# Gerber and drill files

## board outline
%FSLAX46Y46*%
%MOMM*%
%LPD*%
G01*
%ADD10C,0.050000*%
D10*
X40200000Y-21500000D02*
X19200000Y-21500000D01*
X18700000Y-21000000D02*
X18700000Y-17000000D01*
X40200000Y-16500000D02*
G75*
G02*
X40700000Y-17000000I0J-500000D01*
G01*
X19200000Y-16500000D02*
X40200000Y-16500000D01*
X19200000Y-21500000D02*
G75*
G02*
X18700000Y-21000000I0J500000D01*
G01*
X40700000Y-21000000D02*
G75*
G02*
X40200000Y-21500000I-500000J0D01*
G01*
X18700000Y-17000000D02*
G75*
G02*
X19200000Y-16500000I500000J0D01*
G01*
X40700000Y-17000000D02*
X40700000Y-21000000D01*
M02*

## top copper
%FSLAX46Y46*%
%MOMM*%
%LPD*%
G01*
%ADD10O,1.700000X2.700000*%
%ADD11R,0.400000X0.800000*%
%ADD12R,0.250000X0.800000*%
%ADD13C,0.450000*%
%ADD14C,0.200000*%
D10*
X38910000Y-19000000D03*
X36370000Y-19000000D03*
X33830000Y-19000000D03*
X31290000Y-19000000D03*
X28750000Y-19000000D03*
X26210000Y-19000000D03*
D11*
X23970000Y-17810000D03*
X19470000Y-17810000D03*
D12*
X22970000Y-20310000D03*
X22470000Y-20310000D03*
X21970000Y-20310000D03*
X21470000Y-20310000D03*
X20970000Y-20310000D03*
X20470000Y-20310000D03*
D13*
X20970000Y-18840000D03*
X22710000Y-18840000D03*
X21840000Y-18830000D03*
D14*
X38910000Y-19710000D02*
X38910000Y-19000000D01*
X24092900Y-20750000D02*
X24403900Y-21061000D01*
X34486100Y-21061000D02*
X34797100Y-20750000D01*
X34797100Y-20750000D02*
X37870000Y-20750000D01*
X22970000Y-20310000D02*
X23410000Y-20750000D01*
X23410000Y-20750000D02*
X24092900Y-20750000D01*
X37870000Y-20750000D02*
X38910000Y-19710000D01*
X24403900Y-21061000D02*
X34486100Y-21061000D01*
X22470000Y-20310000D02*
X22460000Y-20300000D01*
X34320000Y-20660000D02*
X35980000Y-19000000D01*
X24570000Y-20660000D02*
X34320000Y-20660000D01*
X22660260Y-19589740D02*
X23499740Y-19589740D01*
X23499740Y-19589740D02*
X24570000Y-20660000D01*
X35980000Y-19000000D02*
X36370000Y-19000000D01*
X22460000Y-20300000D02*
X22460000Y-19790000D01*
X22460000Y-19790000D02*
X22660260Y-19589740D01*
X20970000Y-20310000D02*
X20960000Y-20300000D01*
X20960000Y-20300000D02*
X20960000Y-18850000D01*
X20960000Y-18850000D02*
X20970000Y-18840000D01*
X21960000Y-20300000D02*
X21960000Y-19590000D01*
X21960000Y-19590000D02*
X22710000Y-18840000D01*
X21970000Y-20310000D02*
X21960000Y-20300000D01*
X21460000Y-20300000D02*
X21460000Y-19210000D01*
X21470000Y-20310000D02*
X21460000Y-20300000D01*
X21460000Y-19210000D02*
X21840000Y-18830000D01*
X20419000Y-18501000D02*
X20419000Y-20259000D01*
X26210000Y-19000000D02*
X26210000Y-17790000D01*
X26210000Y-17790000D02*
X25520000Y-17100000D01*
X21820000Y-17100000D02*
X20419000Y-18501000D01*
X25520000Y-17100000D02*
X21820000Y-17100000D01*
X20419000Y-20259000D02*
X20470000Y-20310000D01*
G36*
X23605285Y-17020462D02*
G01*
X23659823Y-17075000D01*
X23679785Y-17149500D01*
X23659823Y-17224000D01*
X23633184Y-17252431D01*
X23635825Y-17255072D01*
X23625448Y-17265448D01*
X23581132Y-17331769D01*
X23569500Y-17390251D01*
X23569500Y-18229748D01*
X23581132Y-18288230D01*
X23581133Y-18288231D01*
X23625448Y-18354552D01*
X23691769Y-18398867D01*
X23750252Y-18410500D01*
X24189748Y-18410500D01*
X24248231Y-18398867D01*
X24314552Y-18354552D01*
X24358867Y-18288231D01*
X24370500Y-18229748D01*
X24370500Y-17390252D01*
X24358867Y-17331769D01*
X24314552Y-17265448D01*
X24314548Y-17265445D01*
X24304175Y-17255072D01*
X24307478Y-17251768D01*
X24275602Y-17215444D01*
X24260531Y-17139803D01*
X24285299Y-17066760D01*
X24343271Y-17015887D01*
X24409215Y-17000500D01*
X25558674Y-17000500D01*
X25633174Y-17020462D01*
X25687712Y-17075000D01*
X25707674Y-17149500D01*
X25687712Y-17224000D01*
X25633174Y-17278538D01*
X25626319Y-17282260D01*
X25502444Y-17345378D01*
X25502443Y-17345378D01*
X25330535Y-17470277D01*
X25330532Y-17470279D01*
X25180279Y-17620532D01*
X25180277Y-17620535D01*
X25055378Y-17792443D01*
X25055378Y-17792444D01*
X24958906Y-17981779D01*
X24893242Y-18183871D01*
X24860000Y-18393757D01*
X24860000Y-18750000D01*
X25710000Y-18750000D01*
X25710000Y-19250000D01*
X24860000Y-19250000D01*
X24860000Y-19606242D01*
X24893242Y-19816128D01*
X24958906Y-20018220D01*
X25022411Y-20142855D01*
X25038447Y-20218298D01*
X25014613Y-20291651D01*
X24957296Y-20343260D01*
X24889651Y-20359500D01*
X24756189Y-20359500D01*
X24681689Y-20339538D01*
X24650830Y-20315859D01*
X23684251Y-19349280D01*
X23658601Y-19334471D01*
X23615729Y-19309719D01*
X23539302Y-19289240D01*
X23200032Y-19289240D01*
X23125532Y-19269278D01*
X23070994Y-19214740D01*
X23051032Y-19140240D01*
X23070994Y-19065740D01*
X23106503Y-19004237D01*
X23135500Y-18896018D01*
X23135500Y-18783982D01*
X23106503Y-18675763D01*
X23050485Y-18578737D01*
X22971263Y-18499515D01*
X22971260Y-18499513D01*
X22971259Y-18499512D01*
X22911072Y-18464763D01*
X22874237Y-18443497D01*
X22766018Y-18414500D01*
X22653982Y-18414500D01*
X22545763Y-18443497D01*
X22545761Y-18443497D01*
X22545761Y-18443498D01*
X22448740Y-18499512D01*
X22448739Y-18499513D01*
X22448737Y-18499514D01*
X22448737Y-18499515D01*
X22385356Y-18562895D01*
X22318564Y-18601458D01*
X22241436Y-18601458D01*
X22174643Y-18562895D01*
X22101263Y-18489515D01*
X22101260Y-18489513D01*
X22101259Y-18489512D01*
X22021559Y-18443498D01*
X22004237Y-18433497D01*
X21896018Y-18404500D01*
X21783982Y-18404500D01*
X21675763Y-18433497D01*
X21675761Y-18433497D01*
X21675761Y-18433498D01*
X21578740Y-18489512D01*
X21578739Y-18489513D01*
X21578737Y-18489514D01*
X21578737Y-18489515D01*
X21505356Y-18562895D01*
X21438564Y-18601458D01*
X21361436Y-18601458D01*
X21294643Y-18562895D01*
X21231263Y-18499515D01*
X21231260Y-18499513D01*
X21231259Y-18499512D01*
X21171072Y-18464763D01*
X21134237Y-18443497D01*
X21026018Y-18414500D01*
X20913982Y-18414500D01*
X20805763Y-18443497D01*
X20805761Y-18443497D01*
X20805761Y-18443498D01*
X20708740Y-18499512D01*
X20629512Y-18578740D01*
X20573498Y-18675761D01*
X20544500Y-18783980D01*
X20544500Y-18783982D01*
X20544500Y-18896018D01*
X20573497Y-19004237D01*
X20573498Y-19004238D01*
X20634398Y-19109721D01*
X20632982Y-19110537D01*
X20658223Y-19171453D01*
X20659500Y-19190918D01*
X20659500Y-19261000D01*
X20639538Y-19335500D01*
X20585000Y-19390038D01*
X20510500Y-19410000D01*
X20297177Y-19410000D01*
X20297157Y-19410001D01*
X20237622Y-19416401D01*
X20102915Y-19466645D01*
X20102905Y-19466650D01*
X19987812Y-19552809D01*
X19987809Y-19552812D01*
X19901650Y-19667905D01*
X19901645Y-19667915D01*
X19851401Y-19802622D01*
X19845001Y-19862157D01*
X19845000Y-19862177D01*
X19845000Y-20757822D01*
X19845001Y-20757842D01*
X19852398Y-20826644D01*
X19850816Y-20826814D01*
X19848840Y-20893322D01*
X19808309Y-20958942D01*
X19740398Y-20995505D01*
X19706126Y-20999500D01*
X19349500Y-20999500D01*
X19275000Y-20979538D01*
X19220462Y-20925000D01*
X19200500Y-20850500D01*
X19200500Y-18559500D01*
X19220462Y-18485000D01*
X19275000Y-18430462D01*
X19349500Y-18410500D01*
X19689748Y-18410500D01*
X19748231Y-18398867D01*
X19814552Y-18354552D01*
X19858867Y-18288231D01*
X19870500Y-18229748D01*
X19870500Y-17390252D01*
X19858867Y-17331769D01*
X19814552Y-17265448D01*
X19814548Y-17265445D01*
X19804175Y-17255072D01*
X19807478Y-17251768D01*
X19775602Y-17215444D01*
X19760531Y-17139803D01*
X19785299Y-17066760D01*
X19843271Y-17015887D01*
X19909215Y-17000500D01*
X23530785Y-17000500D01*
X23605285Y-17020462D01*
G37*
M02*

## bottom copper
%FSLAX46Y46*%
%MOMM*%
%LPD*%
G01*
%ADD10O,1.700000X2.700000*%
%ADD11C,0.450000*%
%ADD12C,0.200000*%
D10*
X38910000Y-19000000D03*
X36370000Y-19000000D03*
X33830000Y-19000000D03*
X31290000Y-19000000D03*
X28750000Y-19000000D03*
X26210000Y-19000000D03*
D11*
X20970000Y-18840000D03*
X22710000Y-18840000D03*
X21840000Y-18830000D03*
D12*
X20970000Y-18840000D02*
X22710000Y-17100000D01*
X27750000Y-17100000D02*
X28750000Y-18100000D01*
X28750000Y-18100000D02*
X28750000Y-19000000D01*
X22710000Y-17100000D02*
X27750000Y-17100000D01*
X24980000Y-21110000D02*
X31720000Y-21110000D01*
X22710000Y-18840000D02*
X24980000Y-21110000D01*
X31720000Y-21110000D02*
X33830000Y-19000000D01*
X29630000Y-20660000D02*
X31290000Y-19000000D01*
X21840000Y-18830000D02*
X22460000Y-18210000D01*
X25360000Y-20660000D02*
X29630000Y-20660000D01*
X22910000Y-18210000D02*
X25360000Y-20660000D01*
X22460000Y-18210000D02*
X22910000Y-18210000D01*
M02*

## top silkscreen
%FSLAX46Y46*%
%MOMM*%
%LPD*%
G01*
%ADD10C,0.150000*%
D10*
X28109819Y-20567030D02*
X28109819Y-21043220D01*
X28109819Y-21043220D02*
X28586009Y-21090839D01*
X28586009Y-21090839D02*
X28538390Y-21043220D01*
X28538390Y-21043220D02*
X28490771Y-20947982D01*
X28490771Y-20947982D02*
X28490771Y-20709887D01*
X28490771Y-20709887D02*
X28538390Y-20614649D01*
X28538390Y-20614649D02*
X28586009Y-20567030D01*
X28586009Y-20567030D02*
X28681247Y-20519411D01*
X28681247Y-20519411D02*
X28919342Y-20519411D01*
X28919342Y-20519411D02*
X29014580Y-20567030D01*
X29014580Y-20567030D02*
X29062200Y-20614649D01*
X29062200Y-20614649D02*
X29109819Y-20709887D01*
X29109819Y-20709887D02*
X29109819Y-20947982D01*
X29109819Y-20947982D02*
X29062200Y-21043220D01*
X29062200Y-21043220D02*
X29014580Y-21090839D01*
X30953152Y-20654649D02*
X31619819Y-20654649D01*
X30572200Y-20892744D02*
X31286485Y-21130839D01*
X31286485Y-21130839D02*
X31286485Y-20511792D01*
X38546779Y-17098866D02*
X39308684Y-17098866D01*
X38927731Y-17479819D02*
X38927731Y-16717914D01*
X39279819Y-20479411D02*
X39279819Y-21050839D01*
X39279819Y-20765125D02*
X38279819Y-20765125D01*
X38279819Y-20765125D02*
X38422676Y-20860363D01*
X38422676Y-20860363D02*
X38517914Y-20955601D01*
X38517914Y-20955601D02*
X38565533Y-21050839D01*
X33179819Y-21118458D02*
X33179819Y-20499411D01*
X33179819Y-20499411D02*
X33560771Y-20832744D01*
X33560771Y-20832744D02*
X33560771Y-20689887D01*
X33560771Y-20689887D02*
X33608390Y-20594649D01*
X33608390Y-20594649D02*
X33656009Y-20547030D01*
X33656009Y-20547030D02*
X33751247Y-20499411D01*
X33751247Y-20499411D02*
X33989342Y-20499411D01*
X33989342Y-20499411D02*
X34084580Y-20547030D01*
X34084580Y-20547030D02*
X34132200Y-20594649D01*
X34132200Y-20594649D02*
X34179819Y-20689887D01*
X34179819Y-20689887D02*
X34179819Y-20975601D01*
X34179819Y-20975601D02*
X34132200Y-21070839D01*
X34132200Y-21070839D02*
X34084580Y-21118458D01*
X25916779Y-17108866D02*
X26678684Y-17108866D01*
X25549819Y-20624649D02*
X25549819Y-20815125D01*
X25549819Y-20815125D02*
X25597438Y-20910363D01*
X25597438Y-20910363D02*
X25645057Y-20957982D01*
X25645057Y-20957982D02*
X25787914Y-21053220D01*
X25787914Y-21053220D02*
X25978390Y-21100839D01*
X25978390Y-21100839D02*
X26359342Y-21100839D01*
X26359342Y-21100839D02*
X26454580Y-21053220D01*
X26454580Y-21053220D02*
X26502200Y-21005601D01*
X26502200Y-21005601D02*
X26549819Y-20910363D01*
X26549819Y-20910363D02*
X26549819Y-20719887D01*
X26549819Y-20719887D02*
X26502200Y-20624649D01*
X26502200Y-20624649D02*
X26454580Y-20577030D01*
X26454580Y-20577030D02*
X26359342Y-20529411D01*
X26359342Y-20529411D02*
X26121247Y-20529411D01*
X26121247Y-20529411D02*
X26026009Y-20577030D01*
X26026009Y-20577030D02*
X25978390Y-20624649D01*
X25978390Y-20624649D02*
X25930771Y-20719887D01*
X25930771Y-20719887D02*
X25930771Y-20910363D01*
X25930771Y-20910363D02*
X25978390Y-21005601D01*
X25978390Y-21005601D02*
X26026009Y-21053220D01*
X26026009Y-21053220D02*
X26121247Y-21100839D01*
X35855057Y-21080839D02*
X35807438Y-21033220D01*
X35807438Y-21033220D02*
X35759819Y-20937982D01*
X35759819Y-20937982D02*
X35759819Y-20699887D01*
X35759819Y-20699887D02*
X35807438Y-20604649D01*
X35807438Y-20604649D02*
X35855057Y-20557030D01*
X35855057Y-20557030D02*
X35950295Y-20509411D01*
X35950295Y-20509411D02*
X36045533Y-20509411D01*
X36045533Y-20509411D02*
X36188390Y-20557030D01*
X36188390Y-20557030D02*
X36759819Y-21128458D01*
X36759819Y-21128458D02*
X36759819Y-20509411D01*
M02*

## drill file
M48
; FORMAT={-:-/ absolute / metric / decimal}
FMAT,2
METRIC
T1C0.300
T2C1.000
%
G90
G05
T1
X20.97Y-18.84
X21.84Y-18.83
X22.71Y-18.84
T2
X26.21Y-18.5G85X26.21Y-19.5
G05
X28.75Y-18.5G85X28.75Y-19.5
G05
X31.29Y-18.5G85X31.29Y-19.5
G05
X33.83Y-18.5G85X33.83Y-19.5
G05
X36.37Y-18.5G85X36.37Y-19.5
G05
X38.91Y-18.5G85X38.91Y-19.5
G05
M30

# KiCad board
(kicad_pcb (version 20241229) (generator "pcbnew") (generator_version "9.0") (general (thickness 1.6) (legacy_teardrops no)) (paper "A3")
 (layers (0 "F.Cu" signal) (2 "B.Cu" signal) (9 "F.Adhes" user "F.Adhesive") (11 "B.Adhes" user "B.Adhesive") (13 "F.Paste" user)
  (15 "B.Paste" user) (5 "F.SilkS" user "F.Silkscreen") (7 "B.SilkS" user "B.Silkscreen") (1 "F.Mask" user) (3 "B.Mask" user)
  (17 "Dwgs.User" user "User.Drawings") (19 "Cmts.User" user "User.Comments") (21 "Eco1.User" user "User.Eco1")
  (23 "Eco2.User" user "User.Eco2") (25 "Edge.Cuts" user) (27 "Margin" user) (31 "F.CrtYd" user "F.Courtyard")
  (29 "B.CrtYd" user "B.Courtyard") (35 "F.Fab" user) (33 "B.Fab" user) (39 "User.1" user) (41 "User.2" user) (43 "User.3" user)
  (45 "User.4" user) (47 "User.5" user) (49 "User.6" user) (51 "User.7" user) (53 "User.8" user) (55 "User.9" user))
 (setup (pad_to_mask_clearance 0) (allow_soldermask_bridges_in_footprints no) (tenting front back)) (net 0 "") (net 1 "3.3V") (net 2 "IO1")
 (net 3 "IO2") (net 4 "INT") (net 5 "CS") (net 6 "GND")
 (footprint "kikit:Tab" (layer "F.Cu") (at 37.43 22.22 90)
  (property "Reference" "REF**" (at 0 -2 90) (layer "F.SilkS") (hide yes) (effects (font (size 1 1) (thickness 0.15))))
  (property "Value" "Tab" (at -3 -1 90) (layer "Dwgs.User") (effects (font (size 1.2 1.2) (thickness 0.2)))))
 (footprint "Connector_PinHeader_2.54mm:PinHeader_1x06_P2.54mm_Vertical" (layer "F.Cu") (at 38.91 19 -90)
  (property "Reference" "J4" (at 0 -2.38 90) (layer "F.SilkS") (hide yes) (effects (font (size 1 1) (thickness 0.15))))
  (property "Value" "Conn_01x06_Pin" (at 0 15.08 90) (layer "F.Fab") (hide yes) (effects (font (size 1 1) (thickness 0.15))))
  (pad "1" thru_hole oval (at 0 0 270) (size 2.7 1.7) (drill oval 2 1) (layers "*.Cu" "*.Mask") (remove_unused_layers no) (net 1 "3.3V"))
  (pad "2" thru_hole oval (at 0 2.54 270) (size 2.7 1.7) (drill oval 2 1) (layers "*.Cu" "*.Mask") (remove_unused_layers no) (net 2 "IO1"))
  (pad "3" thru_hole oval (at 0 5.08 270) (size 2.7 1.7) (drill oval 2 1) (layers "*.Cu" "*.Mask") (remove_unused_layers no) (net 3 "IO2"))
  (pad "4" thru_hole oval (at 0 7.62 270) (size 2.7 1.7) (drill oval 2 1) (layers "*.Cu" "*.Mask") (remove_unused_layers no) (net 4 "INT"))
  (pad "5" thru_hole oval (at 0 10.16 270) (size 2.7 1.7) (drill oval 2 1) (layers "*.Cu" "*.Mask") (remove_unused_layers no) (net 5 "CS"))
  (pad "6" thru_hole oval (at 0 12.7 270) (size 2.7 1.7) (drill oval 2 1) (layers "*.Cu" "*.Mask") (remove_unused_layers no) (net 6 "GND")))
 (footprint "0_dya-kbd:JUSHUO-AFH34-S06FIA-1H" (layer "F.Cu") (at 21.72 20.31 180)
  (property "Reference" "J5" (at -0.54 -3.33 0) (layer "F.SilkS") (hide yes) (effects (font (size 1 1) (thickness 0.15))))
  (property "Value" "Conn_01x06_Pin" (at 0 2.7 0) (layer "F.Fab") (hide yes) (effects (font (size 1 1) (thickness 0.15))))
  (pad "0" smd rect (at -2.25 2.5 180) (size 0.4 0.8) (layers "F.Cu" "F.Mask" "F.Paste") (thermal_bridge_angle 45))
  (pad "0" smd rect (at 2.25 2.5 180) (size 0.4 0.8) (layers "F.Cu" "F.Mask" "F.Paste") (thermal_bridge_angle 45))
  (pad "1" smd rect (at -1.25 0 180) (size 0.25 0.8) (layers "F.Cu" "F.Mask" "F.Paste") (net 1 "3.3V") (thermal_bridge_angle 45))
  (pad "2" smd rect (at -0.75 0 180) (size 0.25 0.8) (layers "F.Cu" "F.Mask" "F.Paste") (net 2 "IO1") (thermal_bridge_angle 45))
  (pad "3" smd rect (at -0.25 0 180) (size 0.25 0.8) (layers "F.Cu" "F.Mask" "F.Paste") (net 3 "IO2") (thermal_bridge_angle 45))
  (pad "4" smd rect (at 0.25 0 180) (size 0.25 0.8) (layers "F.Cu" "F.Mask" "F.Paste") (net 4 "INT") (thermal_bridge_angle 45))
  (pad "5" smd rect (at 0.75 0 180) (size 0.25 0.8) (layers "F.Cu" "F.Mask" "F.Paste") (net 5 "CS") (thermal_bridge_angle 45))
  (pad "6" smd rect (at 1.25 0 180) (size 0.25 0.8) (layers "F.Cu" "F.Mask" "F.Paste") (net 6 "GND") (thermal_bridge_angle 45)))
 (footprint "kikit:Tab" (layer "F.Cu") (at 37.43 15.79 -90)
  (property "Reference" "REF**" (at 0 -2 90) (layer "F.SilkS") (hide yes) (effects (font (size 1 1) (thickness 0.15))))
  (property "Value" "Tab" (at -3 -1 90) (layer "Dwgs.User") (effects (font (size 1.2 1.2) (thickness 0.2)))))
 (gr_line (start 40.2 21.5) (end 19.2 21.5) (stroke (width 0.05) (type default)) (layer "Edge.Cuts"))
 (gr_line (start 18.7 21) (end 18.7 17) (stroke (width 0.05) (type default)) (layer "Edge.Cuts"))
 (gr_arc (start 40.2 16.5) (mid 40.553553 16.646447) (end 40.7 17) (stroke (width 0.05) (type default)) (layer "Edge.Cuts"))
 (gr_line (start 19.2 16.5) (end 40.2 16.5) (stroke (width 0.05) (type default)) (layer "Edge.Cuts"))
 (gr_arc (start 19.2 21.5) (mid 18.846447 21.353553) (end 18.7 21) (stroke (width 0.05) (type default)) (layer "Edge.Cuts"))
 (gr_arc (start 40.7 21) (mid 40.553553 21.353553) (end 40.2 21.5) (stroke (width 0.05) (type default)) (layer "Edge.Cuts"))
 (gr_arc (start 18.7 17) (mid 18.846447 16.646447) (end 19.2 16.5) (stroke (width 0.05) (type default)) (layer "Edge.Cuts"))
 (gr_line (start 40.7 17) (end 40.7 21) (stroke (width 0.05) (type default)) (layer "Edge.Cuts"))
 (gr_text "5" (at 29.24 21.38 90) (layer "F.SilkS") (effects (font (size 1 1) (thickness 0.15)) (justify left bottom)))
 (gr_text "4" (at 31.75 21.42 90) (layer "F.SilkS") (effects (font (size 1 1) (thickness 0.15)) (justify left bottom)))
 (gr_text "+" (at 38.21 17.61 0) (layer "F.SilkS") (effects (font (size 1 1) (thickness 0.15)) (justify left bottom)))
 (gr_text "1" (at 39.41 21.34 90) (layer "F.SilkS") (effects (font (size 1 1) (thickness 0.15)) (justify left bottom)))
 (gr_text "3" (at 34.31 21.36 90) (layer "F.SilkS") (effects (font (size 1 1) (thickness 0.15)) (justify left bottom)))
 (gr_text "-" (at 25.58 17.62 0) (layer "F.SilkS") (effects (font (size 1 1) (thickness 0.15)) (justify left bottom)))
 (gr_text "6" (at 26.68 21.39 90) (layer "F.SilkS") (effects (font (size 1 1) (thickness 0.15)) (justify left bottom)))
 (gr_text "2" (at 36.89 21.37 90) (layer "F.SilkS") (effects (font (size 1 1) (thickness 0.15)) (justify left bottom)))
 (segment (start 38.91 19.71) (end 38.91 19) (width 0.2) (layer "F.Cu") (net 1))
 (segment (start 24.0929 20.75) (end 24.4039 21.061) (width 0.2) (layer "F.Cu") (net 1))
 (segment (start 34.4861 21.061) (end 34.7971 20.75) (width 0.2) (layer "F.Cu") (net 1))
 (segment (start 34.7971 20.75) (end 37.87 20.75) (width 0.2) (layer "F.Cu") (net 1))
 (segment (start 22.97 20.31) (end 23.41 20.75) (width 0.2) (layer "F.Cu") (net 1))
 (segment (start 23.41 20.75) (end 24.0929 20.75) (width 0.2) (layer "F.Cu") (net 1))
 (segment (start 37.87 20.75) (end 38.91 19.71) (width 0.2) (layer "F.Cu") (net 1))
 (segment (start 24.4039 21.061) (end 34.4861 21.061) (width 0.2) (layer "F.Cu") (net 1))
 (segment (start 22.47 20.31) (end 22.46 20.3) (width 0.2) (layer "F.Cu") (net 2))
 (segment (start 34.32 20.66) (end 35.98 19) (width 0.2) (layer "F.Cu") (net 2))
 (segment (start 24.57 20.66) (end 34.32 20.66) (width 0.2) (layer "F.Cu") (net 2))
 (segment (start 22.66026 19.58974) (end 23.49974 19.58974) (width 0.2) (layer "F.Cu") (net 2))
 (segment (start 23.49974 19.58974) (end 24.57 20.66) (width 0.2) (layer "F.Cu") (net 2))
 (segment (start 35.98 19) (end 36.37 19) (width 0.2) (layer "F.Cu") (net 2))
 (segment (start 22.46 20.3) (end 22.46 19.79) (width 0.2) (layer "F.Cu") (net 2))
 (segment (start 22.46 19.79) (end 22.66026 19.58974) (width 0.2) (layer "F.Cu") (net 2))
 (segment (start 20.97 20.31) (end 20.96 20.3) (width 0.2) (layer "F.Cu") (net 5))
 (segment (start 20.96 20.3) (end 20.96 18.85) (width 0.2) (layer "F.Cu") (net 5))
 (segment (start 20.96 18.85) (end 20.97 18.84) (width 0.2) (layer "F.Cu") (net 5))
 (via (at 20.97 18.84) (size 0.45) (drill 0.3) (layers "F.Cu" "B.Cu") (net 5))
 (segment (start 20.97 18.84) (end 22.71 17.1) (width 0.2) (layer "B.Cu") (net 5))
 (segment (start 27.75 17.1) (end 28.75 18.1) (width 0.2) (layer "B.Cu") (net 5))
 (segment (start 28.75 18.1) (end 28.75 19) (width 0.2) (layer "B.Cu") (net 5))
 (segment (start 22.71 17.1) (end 27.75 17.1) (width 0.2) (layer "B.Cu") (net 5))
 (segment (start 21.96 20.3) (end 21.96 19.59) (width 0.2) (layer "F.Cu") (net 3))
 (segment (start 21.96 19.59) (end 22.71 18.84) (width 0.2) (layer "F.Cu") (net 3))
 (segment (start 21.97 20.31) (end 21.96 20.3) (width 0.2) (layer "F.Cu") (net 3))
 (via (at 22.71 18.84) (size 0.45) (drill 0.3) (layers "F.Cu" "B.Cu") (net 3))
 (segment (start 24.98 21.11) (end 31.72 21.11) (width 0.2) (layer "B.Cu") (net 3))
 (segment (start 22.71 18.84) (end 24.98 21.11) (width 0.2) (layer "B.Cu") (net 3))
 (segment (start 31.72 21.11) (end 33.83 19) (width 0.2) (layer "B.Cu") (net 3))
 (segment (start 21.46 20.3) (end 21.46 19.21) (width 0.2) (layer "F.Cu") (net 4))
 (segment (start 21.47 20.31) (end 21.46 20.3) (width 0.2) (layer "F.Cu") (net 4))
 (segment (start 21.46 19.21) (end 21.84 18.83) (width 0.2) (layer "F.Cu") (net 4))
 (via (at 21.84 18.83) (size 0.45) (drill 0.3) (layers "F.Cu" "B.Cu") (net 4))
 (segment (start 29.63 20.66) (end 31.29 19) (width 0.2) (layer "B.Cu") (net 4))
 (segment (start 21.84 18.83) (end 22.46 18.21) (width 0.2) (layer "B.Cu") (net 4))
 (segment (start 25.36 20.66) (end 29.63 20.66) (width 0.2) (layer "B.Cu") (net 4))
 (segment (start 22.91 18.21) (end 25.36 20.66) (width 0.2) (layer "B.Cu") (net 4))
 (segment (start 22.46 18.21) (end 22.91 18.21) (width 0.2) (layer "B.Cu") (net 4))
 (segment (start 20.419 18.501) (end 20.419 20.259) (width 0.2) (layer "F.Cu") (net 6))
 (segment (start 26.21 19) (end 26.21 17.79) (width 0.2) (layer "F.Cu") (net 6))
 (segment (start 26.21 17.79) (end 25.52 17.1) (width 0.2) (layer "F.Cu") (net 6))
 (segment (start 21.82 17.1) (end 20.419 18.501) (width 0.2) (layer "F.Cu") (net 6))
 (segment (start 25.52 17.1) (end 21.82 17.1) (width 0.2) (layer "F.Cu") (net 6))
 (segment (start 20.419 20.259) (end 20.47 20.31) (width 0.2) (layer "F.Cu") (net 6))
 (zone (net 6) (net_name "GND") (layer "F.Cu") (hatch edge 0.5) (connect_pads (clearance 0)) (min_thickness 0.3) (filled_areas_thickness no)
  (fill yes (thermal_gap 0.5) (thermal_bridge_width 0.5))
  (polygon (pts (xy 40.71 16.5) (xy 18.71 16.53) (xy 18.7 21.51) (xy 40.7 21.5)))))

